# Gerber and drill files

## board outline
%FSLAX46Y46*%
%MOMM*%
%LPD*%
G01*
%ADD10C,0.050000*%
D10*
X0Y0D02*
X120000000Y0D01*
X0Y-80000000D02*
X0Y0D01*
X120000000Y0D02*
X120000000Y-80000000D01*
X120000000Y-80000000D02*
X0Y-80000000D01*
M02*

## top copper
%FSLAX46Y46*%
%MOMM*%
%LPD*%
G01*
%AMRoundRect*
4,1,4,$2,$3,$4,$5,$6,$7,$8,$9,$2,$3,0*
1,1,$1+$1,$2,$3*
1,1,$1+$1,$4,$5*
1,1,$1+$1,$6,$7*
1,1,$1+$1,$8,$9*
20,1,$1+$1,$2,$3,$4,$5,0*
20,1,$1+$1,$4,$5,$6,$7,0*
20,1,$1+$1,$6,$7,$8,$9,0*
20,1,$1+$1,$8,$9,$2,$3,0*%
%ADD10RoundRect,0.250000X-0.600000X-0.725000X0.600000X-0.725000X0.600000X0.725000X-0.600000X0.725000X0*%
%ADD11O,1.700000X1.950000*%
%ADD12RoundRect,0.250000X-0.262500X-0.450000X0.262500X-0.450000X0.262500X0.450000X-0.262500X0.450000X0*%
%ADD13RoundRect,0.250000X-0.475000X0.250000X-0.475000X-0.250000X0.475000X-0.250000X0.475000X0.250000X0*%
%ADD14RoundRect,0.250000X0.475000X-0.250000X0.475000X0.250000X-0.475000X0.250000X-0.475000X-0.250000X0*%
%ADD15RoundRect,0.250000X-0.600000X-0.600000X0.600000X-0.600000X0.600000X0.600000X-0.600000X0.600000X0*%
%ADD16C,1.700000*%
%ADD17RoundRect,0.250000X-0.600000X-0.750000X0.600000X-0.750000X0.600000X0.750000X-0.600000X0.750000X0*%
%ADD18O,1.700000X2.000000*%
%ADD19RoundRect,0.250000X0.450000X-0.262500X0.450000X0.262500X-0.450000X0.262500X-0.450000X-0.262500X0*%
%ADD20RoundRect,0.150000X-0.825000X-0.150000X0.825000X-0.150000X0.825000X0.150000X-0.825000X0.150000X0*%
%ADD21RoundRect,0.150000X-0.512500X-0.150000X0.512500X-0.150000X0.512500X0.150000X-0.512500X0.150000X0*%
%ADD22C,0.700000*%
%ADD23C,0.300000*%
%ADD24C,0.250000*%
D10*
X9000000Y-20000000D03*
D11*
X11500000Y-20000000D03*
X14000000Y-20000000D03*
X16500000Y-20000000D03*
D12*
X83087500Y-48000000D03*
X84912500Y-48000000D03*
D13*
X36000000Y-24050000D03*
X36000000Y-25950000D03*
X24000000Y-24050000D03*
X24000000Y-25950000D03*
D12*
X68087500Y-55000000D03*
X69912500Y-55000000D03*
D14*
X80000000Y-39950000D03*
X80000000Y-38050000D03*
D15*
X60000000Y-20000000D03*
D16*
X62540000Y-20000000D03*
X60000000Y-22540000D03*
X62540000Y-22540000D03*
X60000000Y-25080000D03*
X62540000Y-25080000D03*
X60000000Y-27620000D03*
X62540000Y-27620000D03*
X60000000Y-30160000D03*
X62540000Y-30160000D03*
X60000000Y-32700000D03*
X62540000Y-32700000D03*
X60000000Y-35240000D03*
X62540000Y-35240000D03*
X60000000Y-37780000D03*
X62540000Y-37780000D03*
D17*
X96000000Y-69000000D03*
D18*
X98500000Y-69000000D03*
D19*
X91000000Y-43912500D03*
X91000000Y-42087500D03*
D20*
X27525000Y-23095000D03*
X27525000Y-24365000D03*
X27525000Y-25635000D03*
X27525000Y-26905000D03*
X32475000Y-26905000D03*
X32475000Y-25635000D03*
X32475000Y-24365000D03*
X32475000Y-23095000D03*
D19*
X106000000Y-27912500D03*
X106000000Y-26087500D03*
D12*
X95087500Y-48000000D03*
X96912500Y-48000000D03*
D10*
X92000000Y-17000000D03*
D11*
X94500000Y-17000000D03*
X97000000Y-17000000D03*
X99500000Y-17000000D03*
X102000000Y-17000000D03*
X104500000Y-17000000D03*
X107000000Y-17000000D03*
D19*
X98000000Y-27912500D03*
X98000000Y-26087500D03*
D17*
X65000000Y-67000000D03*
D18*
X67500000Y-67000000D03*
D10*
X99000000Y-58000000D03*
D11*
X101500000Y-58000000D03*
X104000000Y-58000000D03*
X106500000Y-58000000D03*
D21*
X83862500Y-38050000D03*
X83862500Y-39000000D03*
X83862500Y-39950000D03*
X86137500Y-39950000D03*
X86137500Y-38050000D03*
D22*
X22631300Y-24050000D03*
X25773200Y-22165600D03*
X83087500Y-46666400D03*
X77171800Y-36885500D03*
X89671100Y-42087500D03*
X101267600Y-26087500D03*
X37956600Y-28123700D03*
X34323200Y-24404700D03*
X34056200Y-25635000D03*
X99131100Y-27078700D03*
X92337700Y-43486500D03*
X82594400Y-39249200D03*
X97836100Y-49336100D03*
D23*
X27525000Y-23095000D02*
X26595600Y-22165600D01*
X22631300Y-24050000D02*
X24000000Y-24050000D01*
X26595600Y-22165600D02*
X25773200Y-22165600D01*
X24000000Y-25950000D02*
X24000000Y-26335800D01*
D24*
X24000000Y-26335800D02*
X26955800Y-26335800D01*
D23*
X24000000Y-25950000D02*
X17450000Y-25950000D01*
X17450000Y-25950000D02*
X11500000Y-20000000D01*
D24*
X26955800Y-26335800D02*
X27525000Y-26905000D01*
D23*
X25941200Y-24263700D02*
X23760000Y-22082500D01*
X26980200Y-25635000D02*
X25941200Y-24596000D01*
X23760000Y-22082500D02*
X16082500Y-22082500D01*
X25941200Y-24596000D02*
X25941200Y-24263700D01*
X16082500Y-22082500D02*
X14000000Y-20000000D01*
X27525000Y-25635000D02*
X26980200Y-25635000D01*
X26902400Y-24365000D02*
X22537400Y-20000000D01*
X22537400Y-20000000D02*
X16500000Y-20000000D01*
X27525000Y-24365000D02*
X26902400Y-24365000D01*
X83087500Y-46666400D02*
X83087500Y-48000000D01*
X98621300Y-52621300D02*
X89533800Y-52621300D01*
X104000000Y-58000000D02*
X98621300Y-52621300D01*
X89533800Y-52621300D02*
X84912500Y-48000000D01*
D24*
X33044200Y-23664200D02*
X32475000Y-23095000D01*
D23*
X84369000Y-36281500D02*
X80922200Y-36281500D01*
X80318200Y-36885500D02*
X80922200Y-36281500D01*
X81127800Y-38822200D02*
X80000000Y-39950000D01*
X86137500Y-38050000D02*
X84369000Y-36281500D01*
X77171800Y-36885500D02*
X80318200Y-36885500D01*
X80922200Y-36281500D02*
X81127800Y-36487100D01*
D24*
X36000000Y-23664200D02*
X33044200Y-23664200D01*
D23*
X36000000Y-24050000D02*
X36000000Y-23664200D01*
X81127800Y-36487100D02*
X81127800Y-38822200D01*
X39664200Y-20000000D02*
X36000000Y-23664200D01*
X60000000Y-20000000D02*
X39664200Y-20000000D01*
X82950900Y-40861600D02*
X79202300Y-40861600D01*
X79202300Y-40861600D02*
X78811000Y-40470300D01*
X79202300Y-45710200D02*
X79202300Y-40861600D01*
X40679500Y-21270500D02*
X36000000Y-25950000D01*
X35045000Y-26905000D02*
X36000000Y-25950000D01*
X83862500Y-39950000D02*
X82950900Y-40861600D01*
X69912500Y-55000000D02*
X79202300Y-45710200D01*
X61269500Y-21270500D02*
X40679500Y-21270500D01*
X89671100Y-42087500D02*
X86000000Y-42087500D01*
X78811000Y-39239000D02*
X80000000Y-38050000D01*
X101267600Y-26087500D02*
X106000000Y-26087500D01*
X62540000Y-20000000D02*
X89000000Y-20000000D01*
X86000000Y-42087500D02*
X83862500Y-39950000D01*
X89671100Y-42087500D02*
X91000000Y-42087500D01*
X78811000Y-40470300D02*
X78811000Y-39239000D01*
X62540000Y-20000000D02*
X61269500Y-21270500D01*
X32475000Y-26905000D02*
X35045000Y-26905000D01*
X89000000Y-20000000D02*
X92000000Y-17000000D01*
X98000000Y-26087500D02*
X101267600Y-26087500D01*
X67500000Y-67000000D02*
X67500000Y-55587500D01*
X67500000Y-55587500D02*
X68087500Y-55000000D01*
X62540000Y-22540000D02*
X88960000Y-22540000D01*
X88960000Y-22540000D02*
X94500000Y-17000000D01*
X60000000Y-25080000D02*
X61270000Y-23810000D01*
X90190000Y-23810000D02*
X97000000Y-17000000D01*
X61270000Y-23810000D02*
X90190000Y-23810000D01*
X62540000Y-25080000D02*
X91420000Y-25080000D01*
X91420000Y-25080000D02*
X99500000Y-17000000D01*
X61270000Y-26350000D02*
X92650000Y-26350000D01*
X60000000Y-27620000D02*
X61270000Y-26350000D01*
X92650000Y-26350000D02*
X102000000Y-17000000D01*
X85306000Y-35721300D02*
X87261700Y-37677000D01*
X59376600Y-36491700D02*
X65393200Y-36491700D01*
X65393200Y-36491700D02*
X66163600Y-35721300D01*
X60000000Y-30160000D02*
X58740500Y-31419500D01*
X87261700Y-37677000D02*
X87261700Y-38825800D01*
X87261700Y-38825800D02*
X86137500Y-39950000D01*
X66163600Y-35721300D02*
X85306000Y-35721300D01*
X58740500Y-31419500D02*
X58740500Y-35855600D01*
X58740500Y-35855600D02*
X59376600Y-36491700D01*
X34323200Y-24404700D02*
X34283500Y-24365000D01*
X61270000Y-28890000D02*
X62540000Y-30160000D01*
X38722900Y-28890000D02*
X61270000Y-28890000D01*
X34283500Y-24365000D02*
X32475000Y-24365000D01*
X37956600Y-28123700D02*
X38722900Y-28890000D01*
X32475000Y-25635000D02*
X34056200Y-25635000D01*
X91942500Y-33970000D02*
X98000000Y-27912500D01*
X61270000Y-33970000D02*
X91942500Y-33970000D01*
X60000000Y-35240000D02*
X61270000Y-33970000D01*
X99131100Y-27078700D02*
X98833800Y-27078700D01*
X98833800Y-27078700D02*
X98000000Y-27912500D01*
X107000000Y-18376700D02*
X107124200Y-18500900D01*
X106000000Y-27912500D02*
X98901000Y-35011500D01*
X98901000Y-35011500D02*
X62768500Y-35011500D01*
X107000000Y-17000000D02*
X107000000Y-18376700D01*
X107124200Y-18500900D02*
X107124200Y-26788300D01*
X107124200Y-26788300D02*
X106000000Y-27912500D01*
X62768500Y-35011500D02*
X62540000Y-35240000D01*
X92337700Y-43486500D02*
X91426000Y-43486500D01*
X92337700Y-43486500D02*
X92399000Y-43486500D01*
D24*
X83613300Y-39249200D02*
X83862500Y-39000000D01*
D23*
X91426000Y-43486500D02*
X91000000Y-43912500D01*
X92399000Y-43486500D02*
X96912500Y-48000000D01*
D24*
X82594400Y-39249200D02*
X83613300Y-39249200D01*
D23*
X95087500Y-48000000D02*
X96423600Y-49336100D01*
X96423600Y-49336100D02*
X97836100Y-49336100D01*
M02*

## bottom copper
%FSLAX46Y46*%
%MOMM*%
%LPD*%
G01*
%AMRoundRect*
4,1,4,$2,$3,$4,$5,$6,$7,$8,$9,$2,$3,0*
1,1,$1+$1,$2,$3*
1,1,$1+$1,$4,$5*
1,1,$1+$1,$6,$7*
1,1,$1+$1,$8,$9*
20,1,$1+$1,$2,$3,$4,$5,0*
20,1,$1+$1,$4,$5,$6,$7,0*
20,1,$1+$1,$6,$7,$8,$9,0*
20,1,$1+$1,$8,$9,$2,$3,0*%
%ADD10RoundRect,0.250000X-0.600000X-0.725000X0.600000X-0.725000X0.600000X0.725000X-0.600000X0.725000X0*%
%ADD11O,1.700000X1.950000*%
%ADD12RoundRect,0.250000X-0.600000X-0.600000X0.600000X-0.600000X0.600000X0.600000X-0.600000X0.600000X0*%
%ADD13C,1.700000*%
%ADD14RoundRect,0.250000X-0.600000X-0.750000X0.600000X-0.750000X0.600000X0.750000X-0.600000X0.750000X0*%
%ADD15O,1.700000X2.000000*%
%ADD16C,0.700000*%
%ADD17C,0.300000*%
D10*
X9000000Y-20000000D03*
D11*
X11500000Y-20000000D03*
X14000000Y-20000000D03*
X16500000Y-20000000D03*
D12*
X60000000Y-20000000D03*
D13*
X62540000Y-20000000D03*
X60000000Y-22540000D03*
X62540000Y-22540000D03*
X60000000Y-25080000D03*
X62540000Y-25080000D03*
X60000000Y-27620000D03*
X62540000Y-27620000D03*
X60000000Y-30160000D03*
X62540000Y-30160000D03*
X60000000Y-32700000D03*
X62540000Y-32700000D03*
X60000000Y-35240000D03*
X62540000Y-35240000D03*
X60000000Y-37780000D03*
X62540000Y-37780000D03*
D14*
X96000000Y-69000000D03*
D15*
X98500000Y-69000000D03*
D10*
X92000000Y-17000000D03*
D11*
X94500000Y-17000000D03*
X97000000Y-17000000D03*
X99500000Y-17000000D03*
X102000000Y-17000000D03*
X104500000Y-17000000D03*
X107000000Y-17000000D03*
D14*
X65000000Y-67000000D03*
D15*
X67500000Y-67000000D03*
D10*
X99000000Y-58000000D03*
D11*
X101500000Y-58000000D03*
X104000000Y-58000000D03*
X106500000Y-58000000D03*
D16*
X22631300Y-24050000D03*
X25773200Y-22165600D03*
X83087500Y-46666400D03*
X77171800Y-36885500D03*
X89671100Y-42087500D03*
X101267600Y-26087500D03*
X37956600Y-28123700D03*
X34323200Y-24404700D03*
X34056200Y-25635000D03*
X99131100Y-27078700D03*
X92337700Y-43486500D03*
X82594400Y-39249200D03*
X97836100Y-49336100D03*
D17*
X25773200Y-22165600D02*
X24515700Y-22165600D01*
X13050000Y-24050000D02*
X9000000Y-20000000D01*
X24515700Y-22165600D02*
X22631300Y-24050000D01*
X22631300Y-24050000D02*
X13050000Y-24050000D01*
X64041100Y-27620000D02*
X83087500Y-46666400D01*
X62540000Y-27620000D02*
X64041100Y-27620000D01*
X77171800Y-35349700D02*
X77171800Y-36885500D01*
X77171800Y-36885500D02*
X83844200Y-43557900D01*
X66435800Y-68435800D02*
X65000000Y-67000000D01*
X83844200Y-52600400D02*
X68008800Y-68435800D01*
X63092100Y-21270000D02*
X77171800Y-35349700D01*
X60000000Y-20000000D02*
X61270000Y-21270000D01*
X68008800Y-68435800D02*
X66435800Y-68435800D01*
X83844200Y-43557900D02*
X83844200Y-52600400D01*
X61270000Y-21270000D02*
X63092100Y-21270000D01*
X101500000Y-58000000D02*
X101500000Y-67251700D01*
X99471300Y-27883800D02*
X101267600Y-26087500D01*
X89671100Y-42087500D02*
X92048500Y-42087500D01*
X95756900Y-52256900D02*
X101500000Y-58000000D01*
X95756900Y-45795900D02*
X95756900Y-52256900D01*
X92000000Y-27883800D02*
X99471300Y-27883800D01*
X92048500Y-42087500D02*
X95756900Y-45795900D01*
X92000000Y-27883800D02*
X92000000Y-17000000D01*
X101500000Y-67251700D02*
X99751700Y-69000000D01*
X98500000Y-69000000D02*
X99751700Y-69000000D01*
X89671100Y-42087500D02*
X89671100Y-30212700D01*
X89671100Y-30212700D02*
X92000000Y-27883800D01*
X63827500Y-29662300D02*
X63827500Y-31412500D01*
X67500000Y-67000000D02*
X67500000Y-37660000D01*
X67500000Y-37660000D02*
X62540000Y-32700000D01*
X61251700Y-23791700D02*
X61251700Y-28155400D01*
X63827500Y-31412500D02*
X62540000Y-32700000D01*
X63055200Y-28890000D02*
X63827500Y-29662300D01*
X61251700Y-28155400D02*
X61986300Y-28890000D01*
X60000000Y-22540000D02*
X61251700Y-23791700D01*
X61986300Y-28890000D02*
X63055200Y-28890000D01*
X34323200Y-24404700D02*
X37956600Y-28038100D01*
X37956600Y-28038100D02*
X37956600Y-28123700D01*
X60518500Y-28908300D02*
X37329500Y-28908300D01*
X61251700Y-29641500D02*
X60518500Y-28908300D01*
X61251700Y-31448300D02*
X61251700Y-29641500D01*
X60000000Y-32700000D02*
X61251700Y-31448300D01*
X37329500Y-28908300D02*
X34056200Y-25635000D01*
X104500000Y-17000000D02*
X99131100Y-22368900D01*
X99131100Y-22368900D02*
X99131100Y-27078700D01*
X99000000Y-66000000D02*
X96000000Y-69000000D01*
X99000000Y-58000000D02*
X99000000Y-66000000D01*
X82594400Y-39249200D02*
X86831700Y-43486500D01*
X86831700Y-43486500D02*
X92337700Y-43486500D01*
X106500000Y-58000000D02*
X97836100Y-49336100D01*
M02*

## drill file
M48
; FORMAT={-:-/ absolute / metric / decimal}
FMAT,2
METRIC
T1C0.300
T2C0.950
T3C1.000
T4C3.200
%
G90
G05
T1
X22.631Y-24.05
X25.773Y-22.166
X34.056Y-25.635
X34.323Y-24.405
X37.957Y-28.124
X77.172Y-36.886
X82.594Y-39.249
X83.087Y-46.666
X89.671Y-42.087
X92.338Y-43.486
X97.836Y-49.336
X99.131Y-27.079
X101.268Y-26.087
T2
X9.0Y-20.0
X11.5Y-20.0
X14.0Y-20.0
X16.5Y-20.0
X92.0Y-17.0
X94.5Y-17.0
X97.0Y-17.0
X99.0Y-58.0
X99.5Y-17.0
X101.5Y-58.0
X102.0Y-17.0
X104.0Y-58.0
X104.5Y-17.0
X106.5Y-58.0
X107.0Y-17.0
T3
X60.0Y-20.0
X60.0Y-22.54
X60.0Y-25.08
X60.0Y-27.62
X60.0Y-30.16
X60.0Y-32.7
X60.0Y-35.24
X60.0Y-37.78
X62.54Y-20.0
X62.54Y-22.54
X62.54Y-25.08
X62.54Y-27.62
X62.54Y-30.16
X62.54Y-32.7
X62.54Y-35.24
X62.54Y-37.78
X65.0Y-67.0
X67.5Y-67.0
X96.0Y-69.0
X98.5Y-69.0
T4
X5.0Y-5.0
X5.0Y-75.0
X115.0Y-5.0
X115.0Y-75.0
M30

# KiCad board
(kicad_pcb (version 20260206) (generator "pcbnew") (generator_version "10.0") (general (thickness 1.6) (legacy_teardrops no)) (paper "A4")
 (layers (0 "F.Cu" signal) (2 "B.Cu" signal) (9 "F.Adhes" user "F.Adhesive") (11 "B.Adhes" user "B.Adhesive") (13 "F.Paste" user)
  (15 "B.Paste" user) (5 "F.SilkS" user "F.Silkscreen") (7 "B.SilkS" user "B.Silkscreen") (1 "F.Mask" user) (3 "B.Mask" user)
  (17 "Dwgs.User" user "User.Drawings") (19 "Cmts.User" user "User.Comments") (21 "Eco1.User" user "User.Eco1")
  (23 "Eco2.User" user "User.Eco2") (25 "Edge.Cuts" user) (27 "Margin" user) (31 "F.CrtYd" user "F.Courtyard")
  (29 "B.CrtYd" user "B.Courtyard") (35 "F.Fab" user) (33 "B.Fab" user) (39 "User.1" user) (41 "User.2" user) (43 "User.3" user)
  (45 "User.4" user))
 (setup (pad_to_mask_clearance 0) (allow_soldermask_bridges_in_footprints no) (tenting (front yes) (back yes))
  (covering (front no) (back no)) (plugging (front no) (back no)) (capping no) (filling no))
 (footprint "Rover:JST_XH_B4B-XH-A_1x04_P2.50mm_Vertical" (layer "F.Cu") (at 9 20)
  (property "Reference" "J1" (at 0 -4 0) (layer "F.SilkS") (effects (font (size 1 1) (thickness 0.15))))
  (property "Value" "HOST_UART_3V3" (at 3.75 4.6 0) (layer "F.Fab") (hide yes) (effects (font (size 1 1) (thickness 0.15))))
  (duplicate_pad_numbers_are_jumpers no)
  (pad "1" thru_hole roundrect (at 0 0) (size 1.7 1.95) (drill 0.95) (layers "*.Cu" "*.Mask") (remove_unused_layers no)
   (roundrect_rratio 0.147059) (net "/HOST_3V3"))
  (pad "2" thru_hole oval (at 2.5 0) (size 1.7 1.95) (drill 0.95) (layers "*.Cu" "*.Mask") (remove_unused_layers no) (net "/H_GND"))
  (pad "3" thru_hole oval (at 5 0) (size 1.7 1.95) (drill 0.95) (layers "*.Cu" "*.Mask") (remove_unused_layers no) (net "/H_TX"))
  (pad "4" thru_hole oval (at 7.5 0) (size 1.7 1.95) (drill 0.95) (layers "*.Cu" "*.Mask") (remove_unused_layers no) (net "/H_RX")))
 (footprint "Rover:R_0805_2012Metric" (layer "F.Cu") (at 84 48)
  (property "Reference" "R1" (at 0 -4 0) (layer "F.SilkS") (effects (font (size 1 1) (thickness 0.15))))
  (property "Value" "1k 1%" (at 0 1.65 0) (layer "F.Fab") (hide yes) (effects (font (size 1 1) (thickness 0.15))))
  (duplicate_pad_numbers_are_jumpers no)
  (pad "1" smd roundrect (at -0.9125 0) (size 1.025 1.4) (layers "F.Cu" "F.Mask" "F.Paste") (roundrect_rratio 0.243902) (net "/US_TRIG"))
  (pad "2" smd roundrect (at 0.9125 0) (size 1.025 1.4) (layers "F.Cu" "F.Mask" "F.Paste") (roundrect_rratio 0.243902) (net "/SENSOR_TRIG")))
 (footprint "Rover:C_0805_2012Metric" (layer "F.Cu") (at 36 25 -90)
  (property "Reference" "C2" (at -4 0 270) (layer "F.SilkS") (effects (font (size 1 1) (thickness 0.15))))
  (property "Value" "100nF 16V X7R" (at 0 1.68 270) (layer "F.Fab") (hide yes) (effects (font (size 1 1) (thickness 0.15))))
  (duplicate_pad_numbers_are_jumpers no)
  (pad "1" smd roundrect (at -0.95 0 270) (size 1 1.45) (layers "F.Cu" "F.Mask" "F.Paste") (roundrect_rratio 0.25) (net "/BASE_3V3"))
  (pad "2" smd roundrect (at 0.95 0 270) (size 1 1.45) (layers "F.Cu" "F.Mask" "F.Paste") (roundrect_rratio 0.25) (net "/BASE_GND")))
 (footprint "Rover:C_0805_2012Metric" (layer "F.Cu") (at 24 25 -90)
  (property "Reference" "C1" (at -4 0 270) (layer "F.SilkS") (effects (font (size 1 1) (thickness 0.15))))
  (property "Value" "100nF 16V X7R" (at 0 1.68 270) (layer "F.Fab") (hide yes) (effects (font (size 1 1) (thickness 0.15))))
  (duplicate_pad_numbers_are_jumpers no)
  (pad "1" smd roundrect (at -0.95 0 270) (size 1 1.45) (layers "F.Cu" "F.Mask" "F.Paste") (roundrect_rratio 0.25) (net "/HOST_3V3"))
  (pad "2" smd roundrect (at 0.95 0 270) (size 1 1.45) (layers "F.Cu" "F.Mask" "F.Paste") (roundrect_rratio 0.25) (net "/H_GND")))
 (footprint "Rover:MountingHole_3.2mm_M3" (layer "F.Cu") (at 115 75)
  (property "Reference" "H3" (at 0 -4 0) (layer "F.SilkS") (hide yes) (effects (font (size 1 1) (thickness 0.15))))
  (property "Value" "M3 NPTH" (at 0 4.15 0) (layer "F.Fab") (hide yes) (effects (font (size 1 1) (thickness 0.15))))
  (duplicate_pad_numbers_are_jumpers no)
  (pad "" np_thru_hole circle (at 0 0) (size 3.2 3.2) (drill 3.2) (layers "*.Cu" "*.Mask")))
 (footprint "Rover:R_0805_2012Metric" (layer "F.Cu") (at 69 55)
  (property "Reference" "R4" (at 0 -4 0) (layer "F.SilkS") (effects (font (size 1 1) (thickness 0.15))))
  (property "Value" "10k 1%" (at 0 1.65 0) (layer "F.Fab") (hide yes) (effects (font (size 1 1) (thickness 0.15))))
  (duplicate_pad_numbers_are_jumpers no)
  (pad "1" smd roundrect (at -0.9125 0) (size 1.025 1.4) (layers "F.Cu" "F.Mask" "F.Paste") (roundrect_rratio 0.243902) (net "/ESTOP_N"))
  (pad "2" smd roundrect (at 0.9125 0) (size 1.025 1.4) (layers "F.Cu" "F.Mask" "F.Paste") (roundrect_rratio 0.243902) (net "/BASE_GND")))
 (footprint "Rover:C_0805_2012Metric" (layer "F.Cu") (at 80 39 90)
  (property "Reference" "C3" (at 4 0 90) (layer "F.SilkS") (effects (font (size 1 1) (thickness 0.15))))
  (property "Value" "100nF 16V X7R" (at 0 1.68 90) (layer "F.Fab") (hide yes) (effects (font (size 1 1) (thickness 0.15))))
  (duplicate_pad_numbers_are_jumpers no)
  (pad "1" smd roundrect (at -0.95 0 90) (size 1 1.45) (layers "F.Cu" "F.Mask" "F.Paste") (roundrect_rratio 0.25) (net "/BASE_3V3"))
  (pad "2" smd roundrect (at 0.95 0 90) (size 1 1.45) (layers "F.Cu" "F.Mask" "F.Paste") (roundrect_rratio 0.25) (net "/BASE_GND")))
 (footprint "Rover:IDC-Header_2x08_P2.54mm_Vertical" (layer "F.Cu") (at 60 20)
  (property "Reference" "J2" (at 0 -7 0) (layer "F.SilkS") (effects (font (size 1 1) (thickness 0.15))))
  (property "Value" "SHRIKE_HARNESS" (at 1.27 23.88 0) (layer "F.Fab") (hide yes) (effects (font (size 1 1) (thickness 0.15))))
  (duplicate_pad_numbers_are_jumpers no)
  (pad "1" thru_hole roundrect (at 0 0) (size 1.7 1.7) (drill 1) (layers "*.Cu" "*.Mask") (remove_unused_layers no)
   (roundrect_rratio 0.147059) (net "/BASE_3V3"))
  (pad "2" thru_hole circle (at 2.54 0) (size 1.7 1.7) (drill 1) (layers "*.Cu" "*.Mask") (remove_unused_layers no) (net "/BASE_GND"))
  (pad "3" thru_hole circle (at 0 2.54) (size 1.7 1.7) (drill 1) (layers "*.Cu" "*.Mask") (remove_unused_layers no) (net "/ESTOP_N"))
  (pad "4" thru_hole circle (at 2.54 2.54) (size 1.7 1.7) (drill 1) (layers "*.Cu" "*.Mask") (remove_unused_layers no) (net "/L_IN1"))
  (pad "5" thru_hole circle (at 0 5.08) (size 1.7 1.7) (drill 1) (layers "*.Cu" "*.Mask") (remove_unused_layers no) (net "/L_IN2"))
  (pad "6" thru_hole circle (at 2.54 5.08) (size 1.7 1.7) (drill 1) (layers "*.Cu" "*.Mask") (remove_unused_layers no) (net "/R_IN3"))
  (pad "7" thru_hole circle (at 0 7.62) (size 1.7 1.7) (drill 1) (layers "*.Cu" "*.Mask") (remove_unused_layers no) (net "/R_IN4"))
  (pad "8" thru_hole circle (at 2.54 7.62) (size 1.7 1.7) (drill 1) (layers "*.Cu" "*.Mask") (remove_unused_layers no) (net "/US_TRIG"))
  (pad "9" thru_hole circle (at 0 10.16) (size 1.7 1.7) (drill 1) (layers "*.Cu" "*.Mask") (remove_unused_layers no) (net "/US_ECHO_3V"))
  (pad "10" thru_hole circle (at 2.54 10.16) (size 1.7 1.7) (drill 1) (layers "*.Cu" "*.Mask") (remove_unused_layers no) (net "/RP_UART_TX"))
  (pad "11" thru_hole circle (at 0 12.7) (size 1.7 1.7) (drill 1) (layers "*.Cu" "*.Mask") (remove_unused_layers no) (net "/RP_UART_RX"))
  (pad "12" thru_hole circle (at 2.54 12.7) (size 1.7 1.7) (drill 1) (layers "*.Cu" "*.Mask") (remove_unused_layers no) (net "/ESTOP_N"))
  (pad "13" thru_hole circle (at 0 15.24) (size 1.7 1.7) (drill 1) (layers "*.Cu" "*.Mask") (remove_unused_layers no) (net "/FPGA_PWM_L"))
  (pad "14" thru_hole circle (at 2.54 15.24) (size 1.7 1.7) (drill 1) (layers "*.Cu" "*.Mask") (remove_unused_layers no) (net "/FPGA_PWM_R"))
  (pad "15" thru_hole circle (at 0 17.78) (size 1.7 1.7) (drill 1) (layers "*.Cu" "*.Mask") (remove_unused_layers no)
   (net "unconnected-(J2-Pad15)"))
  (pad "16" thru_hole circle (at 2.54 17.78) (size 1.7 1.7) (drill 1) (layers "*.Cu" "*.Mask") (remove_unused_layers no)
   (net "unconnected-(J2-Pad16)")))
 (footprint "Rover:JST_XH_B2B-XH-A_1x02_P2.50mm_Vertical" (layer "F.Cu") (at 96 69)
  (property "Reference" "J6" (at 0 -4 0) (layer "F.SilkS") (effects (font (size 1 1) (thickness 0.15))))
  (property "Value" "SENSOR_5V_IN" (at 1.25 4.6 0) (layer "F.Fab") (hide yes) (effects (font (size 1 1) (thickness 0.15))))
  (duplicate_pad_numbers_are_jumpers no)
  (pad "1" thru_hole roundrect (at 0 0) (size 1.7 2) (drill 1) (layers "*.Cu" "*.Mask") (remove_unused_layers no)
   (roundrect_rratio 0.147059) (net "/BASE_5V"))
  (pad "2" thru_hole oval (at 2.5 0) (size 1.7 2) (drill 1) (layers "*.Cu" "*.Mask") (remove_unused_layers no) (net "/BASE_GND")))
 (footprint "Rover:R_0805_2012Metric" (layer "F.Cu") (at 91 43 90)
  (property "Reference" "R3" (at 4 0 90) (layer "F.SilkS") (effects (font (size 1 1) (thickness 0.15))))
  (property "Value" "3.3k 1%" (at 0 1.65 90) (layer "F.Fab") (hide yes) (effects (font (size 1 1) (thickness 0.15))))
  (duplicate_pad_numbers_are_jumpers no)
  (pad "1" smd roundrect (at -0.9125 0 90) (size 1.025 1.4) (layers "F.Cu" "F.Mask" "F.Paste") (roundrect_rratio 0.243902) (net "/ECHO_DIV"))
  (pad "2" smd roundrect (at 0.9125 0 90) (size 1.025 1.4) (layers "F.Cu" "F.Mask" "F.Paste") (roundrect_rratio 0.243902) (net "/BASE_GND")))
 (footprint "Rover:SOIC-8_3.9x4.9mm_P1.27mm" (layer "F.Cu") (at 30 25)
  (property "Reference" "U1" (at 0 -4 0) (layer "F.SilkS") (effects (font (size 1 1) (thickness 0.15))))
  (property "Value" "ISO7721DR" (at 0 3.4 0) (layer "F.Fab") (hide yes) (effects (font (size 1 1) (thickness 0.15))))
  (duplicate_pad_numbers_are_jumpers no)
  (pad "1" smd roundrect (at -2.475 -1.905) (size 1.95 0.6) (layers "F.Cu" "F.Mask" "F.Paste") (roundrect_rratio 0.25) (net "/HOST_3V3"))
  (pad "2" smd roundrect (at -2.475 -0.635) (size 1.95 0.6) (layers "F.Cu" "F.Mask" "F.Paste") (roundrect_rratio 0.25) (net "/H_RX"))
  (pad "3" smd roundrect (at -2.475 0.635) (size 1.95 0.6) (layers "F.Cu" "F.Mask" "F.Paste") (roundrect_rratio 0.25) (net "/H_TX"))
  (pad "4" smd roundrect (at -2.475 1.905) (size 1.95 0.6) (layers "F.Cu" "F.Mask" "F.Paste") (roundrect_rratio 0.25) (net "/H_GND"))
  (pad "5" smd roundrect (at 2.475 1.905) (size 1.95 0.6) (layers "F.Cu" "F.Mask" "F.Paste") (roundrect_rratio 0.25) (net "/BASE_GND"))
  (pad "6" smd roundrect (at 2.475 0.635) (size 1.95 0.6) (layers "F.Cu" "F.Mask" "F.Paste") (roundrect_rratio 0.25) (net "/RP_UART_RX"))
  (pad "7" smd roundrect (at 2.475 -0.635) (size 1.95 0.6) (layers "F.Cu" "F.Mask" "F.Paste") (roundrect_rratio 0.25) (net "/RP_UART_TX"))
  (pad "8" smd roundrect (at 2.475 -1.905) (size 1.95 0.6) (layers "F.Cu" "F.Mask" "F.Paste") (roundrect_rratio 0.25) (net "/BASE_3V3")))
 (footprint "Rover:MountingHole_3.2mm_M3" (layer "F.Cu") (at 5 75)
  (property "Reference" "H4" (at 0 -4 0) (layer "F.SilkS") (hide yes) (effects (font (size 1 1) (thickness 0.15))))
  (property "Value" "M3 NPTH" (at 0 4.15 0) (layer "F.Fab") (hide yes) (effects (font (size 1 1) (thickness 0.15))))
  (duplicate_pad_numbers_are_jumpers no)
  (pad "" np_thru_hole circle (at 0 0) (size 3.2 3.2) (drill 3.2) (layers "*.Cu" "*.Mask")))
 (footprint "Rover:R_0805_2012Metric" (layer "F.Cu") (at 106 27 90)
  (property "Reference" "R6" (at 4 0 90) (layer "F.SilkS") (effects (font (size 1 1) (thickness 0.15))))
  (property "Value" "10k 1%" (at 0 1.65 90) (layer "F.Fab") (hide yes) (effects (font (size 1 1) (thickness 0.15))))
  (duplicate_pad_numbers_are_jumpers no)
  (pad "1" smd roundrect (at -0.9125 0 90) (size 1.025 1.4) (layers "F.Cu" "F.Mask" "F.Paste") (roundrect_rratio 0.243902)
   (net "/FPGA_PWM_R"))
  (pad "2" smd roundrect (at 0.9125 0 90) (size 1.025 1.4) (layers "F.Cu" "F.Mask" "F.Paste") (roundrect_rratio 0.243902) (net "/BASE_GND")))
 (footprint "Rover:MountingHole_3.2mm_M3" (layer "F.Cu") (at 5 5)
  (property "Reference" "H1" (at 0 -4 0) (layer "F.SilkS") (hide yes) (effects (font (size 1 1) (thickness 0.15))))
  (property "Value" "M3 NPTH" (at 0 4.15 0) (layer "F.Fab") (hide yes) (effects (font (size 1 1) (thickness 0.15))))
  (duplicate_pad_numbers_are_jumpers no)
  (pad "" np_thru_hole circle (at 0 0) (size 3.2 3.2) (drill 3.2) (layers "*.Cu" "*.Mask")))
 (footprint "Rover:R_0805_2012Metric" (layer "F.Cu") (at 96 48)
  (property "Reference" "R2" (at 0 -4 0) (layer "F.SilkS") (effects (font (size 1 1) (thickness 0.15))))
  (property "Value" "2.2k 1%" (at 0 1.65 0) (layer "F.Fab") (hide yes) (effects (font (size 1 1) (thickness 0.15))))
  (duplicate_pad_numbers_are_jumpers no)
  (pad "1" smd roundrect (at -0.9125 0) (size 1.025 1.4) (layers "F.Cu" "F.Mask" "F.Paste") (roundrect_rratio 0.243902) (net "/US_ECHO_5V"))
  (pad "2" smd roundrect (at 0.9125 0) (size 1.025 1.4) (layers "F.Cu" "F.Mask" "F.Paste") (roundrect_rratio 0.243902) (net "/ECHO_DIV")))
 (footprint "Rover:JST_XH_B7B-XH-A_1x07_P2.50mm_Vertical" (layer "F.Cu") (at 92 17)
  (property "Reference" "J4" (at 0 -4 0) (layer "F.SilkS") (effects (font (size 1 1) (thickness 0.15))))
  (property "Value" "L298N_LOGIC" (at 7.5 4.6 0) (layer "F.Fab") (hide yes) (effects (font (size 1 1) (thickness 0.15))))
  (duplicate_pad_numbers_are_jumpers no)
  (pad "1" thru_hole roundrect (at 0 0) (size 1.7 1.95) (drill 0.95) (layers "*.Cu" "*.Mask") (remove_unused_layers no)
   (roundrect_rratio 0.147059) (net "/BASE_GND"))
  (pad "2" thru_hole oval (at 2.5 0) (size 1.7 1.95) (drill 0.95) (layers "*.Cu" "*.Mask") (remove_unused_layers no) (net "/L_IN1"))
  (pad "3" thru_hole oval (at 5 0) (size 1.7 1.95) (drill 0.95) (layers "*.Cu" "*.Mask") (remove_unused_layers no) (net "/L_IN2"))
  (pad "4" thru_hole oval (at 7.5 0) (size 1.7 1.95) (drill 0.95) (layers "*.Cu" "*.Mask") (remove_unused_layers no) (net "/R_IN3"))
  (pad "5" thru_hole oval (at 10 0) (size 1.7 1.95) (drill 0.95) (layers "*.Cu" "*.Mask") (remove_unused_layers no) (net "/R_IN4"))
  (pad "6" thru_hole oval (at 12.5 0) (size 1.7 1.95) (drill 0.95) (layers "*.Cu" "*.Mask") (remove_unused_layers no) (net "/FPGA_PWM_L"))
  (pad "7" thru_hole oval (at 15 0) (size 1.7 1.95) (drill 0.95) (layers "*.Cu" "*.Mask") (remove_unused_layers no) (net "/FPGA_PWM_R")))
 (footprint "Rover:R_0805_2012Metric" (layer "F.Cu") (at 98 27 90)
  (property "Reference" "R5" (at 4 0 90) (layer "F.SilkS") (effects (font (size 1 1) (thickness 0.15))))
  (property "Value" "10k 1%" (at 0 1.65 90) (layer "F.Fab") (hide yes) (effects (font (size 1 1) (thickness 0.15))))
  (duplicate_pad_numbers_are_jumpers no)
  (pad "1" smd roundrect (at -0.9125 0 90) (size 1.025 1.4) (layers "F.Cu" "F.Mask" "F.Paste") (roundrect_rratio 0.243902)
   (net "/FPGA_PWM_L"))
  (pad "2" smd roundrect (at 0.9125 0 90) (size 1.025 1.4) (layers "F.Cu" "F.Mask" "F.Paste") (roundrect_rratio 0.243902) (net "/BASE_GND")))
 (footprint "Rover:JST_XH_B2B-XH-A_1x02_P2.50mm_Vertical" (layer "F.Cu") (at 65 67)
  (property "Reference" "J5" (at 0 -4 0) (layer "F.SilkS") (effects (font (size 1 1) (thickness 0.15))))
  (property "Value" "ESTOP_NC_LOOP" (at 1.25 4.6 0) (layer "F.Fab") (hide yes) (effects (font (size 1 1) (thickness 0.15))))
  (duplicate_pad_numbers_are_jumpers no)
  (pad "1" thru_hole roundrect (at 0 0) (size 1.7 2) (drill 1) (layers "*.Cu" "*.Mask") (remove_unused_layers no)
   (roundrect_rratio 0.147059) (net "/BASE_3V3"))
  (pad "2" thru_hole oval (at 2.5 0) (size 1.7 2) (drill 1) (layers "*.Cu" "*.Mask") (remove_unused_layers no) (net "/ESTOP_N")))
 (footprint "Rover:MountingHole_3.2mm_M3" (layer "F.Cu") (at 115 5)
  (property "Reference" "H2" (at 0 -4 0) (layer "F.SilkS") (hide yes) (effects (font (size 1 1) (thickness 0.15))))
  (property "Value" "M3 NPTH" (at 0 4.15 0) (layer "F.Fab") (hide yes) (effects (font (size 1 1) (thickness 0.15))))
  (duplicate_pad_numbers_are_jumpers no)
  (pad "" np_thru_hole circle (at 0 0) (size 3.2 3.2) (drill 3.2) (layers "*.Cu" "*.Mask")))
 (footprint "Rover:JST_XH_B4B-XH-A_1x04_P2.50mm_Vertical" (layer "F.Cu") (at 99 58)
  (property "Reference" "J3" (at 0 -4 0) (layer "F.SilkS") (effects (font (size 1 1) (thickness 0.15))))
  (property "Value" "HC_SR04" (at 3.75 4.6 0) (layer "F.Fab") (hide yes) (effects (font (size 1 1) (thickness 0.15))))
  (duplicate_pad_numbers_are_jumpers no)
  (pad "1" thru_hole roundrect (at 0 0) (size 1.7 1.95) (drill 0.95) (layers "*.Cu" "*.Mask") (remove_unused_layers no)
   (roundrect_rratio 0.147059) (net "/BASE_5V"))
  (pad "2" thru_hole oval (at 2.5 0) (size 1.7 1.95) (drill 0.95) (layers "*.Cu" "*.Mask") (remove_unused_layers no) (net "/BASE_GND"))
  (pad "3" thru_hole oval (at 5 0) (size 1.7 1.95) (drill 0.95) (layers "*.Cu" "*.Mask") (remove_unused_layers no) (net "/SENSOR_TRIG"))
  (pad "4" thru_hole oval (at 7.5 0) (size 1.7 1.95) (drill 0.95) (layers "*.Cu" "*.Mask") (remove_unused_layers no) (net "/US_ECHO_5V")))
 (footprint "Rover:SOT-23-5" (layer "F.Cu") (at 85 39)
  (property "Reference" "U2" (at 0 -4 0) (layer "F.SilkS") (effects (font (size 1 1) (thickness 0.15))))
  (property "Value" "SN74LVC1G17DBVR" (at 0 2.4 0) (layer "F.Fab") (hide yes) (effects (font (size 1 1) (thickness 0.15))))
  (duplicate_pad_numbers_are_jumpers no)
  (pad "1" smd roundrect (at -1.1375 -0.95) (size 1.325 0.6) (layers "F.Cu" "F.Mask" "F.Paste") (roundrect_rratio 0.25)
   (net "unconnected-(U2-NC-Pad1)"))
  (pad "2" smd roundrect (at -1.1375 0) (size 1.325 0.6) (layers "F.Cu" "F.Mask" "F.Paste") (roundrect_rratio 0.25) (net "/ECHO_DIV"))
  (pad "3" smd roundrect (at -1.1375 0.95) (size 1.325 0.6) (layers "F.Cu" "F.Mask" "F.Paste") (roundrect_rratio 0.25) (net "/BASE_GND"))
  (pad "4" smd roundrect (at 1.1375 0.95) (size 1.325 0.6) (layers "F.Cu" "F.Mask" "F.Paste") (roundrect_rratio 0.25) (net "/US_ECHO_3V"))
  (pad "5" smd roundrect (at 1.1375 -0.95) (size 1.325 0.6) (layers "F.Cu" "F.Mask" "F.Paste") (roundrect_rratio 0.25) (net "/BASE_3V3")))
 (gr_line (start 0 0) (end 120 0) (stroke (width 0.05) (type default)) (layer "Edge.Cuts"))
 (gr_line (start 0 80) (end 0 0) (stroke (width 0.05) (type default)) (layer "Edge.Cuts"))
 (gr_line (start 120 0) (end 120 80) (stroke (width 0.05) (type default)) (layer "Edge.Cuts"))
 (gr_line (start 120 80) (end 0 80) (stroke (width 0.05) (type default)) (layer "Edge.Cuts"))
 (segment (start 27.525 23.095) (end 26.5956 22.1656) (width 0.3) (layer "F.Cu") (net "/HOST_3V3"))
 (segment (start 22.6313 24.05) (end 24 24.05) (width 0.3) (layer "F.Cu") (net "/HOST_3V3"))
 (segment (start 26.5956 22.1656) (end 25.7732 22.1656) (width 0.3) (layer "F.Cu") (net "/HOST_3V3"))
 (via (at 22.6313 24.05) (size 0.7) (drill 0.3) (layers "F.Cu" "B.Cu") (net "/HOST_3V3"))
 (via (at 25.7732 22.1656) (size 0.7) (drill 0.3) (layers "F.Cu" "B.Cu") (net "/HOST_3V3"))
 (segment (start 25.7732 22.1656) (end 24.5157 22.1656) (width 0.3) (layer "B.Cu") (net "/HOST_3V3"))
 (segment (start 13.05 24.05) (end 9 20) (width 0.3) (layer "B.Cu") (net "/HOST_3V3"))
 (segment (start 24.5157 22.1656) (end 22.6313 24.05) (width 0.3) (layer "B.Cu") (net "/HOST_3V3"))
 (segment (start 22.6313 24.05) (end 13.05 24.05) (width 0.3) (layer "B.Cu") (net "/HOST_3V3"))
 (segment (start 24 25.95) (end 24 26.3358) (width 0.3) (layer "F.Cu") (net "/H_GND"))
 (segment (start 24 26.3358) (end 26.9558 26.3358) (width 0.25) (layer "F.Cu") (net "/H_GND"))
 (segment (start 24 25.95) (end 17.45 25.95) (width 0.3) (layer "F.Cu") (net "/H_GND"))
 (segment (start 17.45 25.95) (end 11.5 20) (width 0.3) (layer "F.Cu") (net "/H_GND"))
 (segment (start 26.9558 26.3358) (end 27.525 26.905) (width 0.25) (layer "F.Cu") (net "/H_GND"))
 (segment (start 25.9412 24.2637) (end 23.76 22.0825) (width 0.3) (layer "F.Cu") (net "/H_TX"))
 (segment (start 26.9802 25.635) (end 25.9412 24.596) (width 0.3) (layer "F.Cu") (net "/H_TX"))
 (segment (start 23.76 22.0825) (end 16.0825 22.0825) (width 0.3) (layer "F.Cu") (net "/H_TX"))
 (segment (start 25.9412 24.596) (end 25.9412 24.2637) (width 0.3) (layer "F.Cu") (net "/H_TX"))
 (segment (start 16.0825 22.0825) (end 14 20) (width 0.3) (layer "F.Cu") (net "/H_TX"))
 (segment (start 27.525 25.635) (end 26.9802 25.635) (width 0.3) (layer "F.Cu") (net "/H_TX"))
 (segment (start 26.9024 24.365) (end 22.5374 20) (width 0.3) (layer "F.Cu") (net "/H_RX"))
 (segment (start 22.5374 20) (end 16.5 20) (width 0.3) (layer "F.Cu") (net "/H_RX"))
 (segment (start 27.525 24.365) (end 26.9024 24.365) (width 0.3) (layer "F.Cu") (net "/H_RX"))
 (segment (start 83.0875 46.6664) (end 83.0875 48) (width 0.3) (layer "F.Cu") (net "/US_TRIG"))
 (via (at 83.0875 46.6664) (size 0.7) (drill 0.3) (layers "F.Cu" "B.Cu") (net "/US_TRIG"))
 (segment (start 64.0411 27.62) (end 83.0875 46.6664) (width 0.3) (layer "B.Cu") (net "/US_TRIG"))
 (segment (start 62.54 27.62) (end 64.0411 27.62) (width 0.3) (layer "B.Cu") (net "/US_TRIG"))
 (segment (start 98.6213 52.6213) (end 89.5338 52.6213) (width 0.3) (layer "F.Cu") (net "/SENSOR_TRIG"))
 (segment (start 104 58) (end 98.6213 52.6213) (width 0.3) (layer "F.Cu") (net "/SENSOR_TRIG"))
 (segment (start 89.5338 52.6213) (end 84.9125 48) (width 0.3) (layer "F.Cu") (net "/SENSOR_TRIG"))
 (segment (start 33.0442 23.6642) (end 32.475 23.095) (width 0.25) (layer "F.Cu") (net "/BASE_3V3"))
 (segment (start 84.369 36.2815) (end 80.9222 36.2815) (width 0.3) (layer "F.Cu") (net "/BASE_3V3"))
 (segment (start 80.3182 36.8855) (end 80.9222 36.2815) (width 0.3) (layer "F.Cu") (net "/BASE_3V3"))
 (segment (start 81.1278 38.8222) (end 80 39.95) (width 0.3) (layer "F.Cu") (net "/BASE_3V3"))
 (segment (start 86.1375 38.05) (end 84.369 36.2815) (width 0.3) (layer "F.Cu") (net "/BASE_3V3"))
 (segment (start 77.1718 36.8855) (end 80.3182 36.8855) (width 0.3) (layer "F.Cu") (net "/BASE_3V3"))
 (segment (start 80.9222 36.2815) (end 81.1278 36.4871) (width 0.3) (layer "F.Cu") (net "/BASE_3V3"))
 (segment (start 36 23.6642) (end 33.0442 23.6642) (width 0.25) (layer "F.Cu") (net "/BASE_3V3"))
 (segment (start 36 24.05) (end 36 23.6642) (width 0.3) (layer "F.Cu") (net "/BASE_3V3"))
 (segment (start 81.1278 36.4871) (end 81.1278 38.8222) (width 0.3) (layer "F.Cu") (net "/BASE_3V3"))
 (segment (start 39.6642 20) (end 36 23.6642) (width 0.3) (layer "F.Cu") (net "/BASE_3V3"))
 (segment (start 60 20) (end 39.6642 20) (width 0.3) (layer "F.Cu") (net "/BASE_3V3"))
 (via (at 77.1718 36.8855) (size 0.7) (drill 0.3) (layers "F.Cu" "B.Cu") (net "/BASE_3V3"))
 (segment (start 77.1718 35.3497) (end 77.1718 36.8855) (width 0.3) (layer "B.Cu") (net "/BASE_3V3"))
 (segment (start 77.1718 36.8855) (end 83.8442 43.5579) (width 0.3) (layer "B.Cu") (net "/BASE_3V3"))
 (segment (start 66.4358 68.4358) (end 65 67) (width 0.3) (layer "B.Cu") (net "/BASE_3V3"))
 (segment (start 83.8442 52.6004) (end 68.0088 68.4358) (width 0.3) (layer "B.Cu") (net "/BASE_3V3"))
 (segment (start 63.0921 21.27) (end 77.1718 35.3497) (width 0.3) (layer "B.Cu") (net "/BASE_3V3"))
 (segment (start 60 20) (end 61.27 21.27) (width 0.3) (layer "B.Cu") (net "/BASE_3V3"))
 (segment (start 68.0088 68.4358) (end 66.4358 68.4358) (width 0.3) (layer "B.Cu") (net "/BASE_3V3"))
 (segment (start 83.8442 43.5579) (end 83.8442 52.6004) (width 0.3) (layer "B.Cu") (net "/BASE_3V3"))
 (segment (start 61.27 21.27) (end 63.0921 21.27) (width 0.3) (layer "B.Cu") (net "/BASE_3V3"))
 (segment (start 82.9509 40.8616) (end 79.2023 40.8616) (width 0.3) (layer "F.Cu") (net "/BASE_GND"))
 (segment (start 79.2023 40.8616) (end 78.811 40.4703) (width 0.3) (layer "F.Cu") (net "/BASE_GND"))
 (segment (start 79.2023 45.7102) (end 79.2023 40.8616) (width 0.3) (layer "F.Cu") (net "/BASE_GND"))
 (segment (start 40.6795 21.2705) (end 36 25.95) (width 0.3) (layer "F.Cu") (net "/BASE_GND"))
 (segment (start 35.045 26.905) (end 36 25.95) (width 0.3) (layer "F.Cu") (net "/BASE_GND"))
 (segment (start 83.8625 39.95) (end 82.9509 40.8616) (width 0.3) (layer "F.Cu") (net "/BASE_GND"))
 (segment (start 69.9125 55) (end 79.2023 45.7102) (width 0.3) (layer "F.Cu") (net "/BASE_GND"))
 (segment (start 61.2695 21.2705) (end 40.6795 21.2705) (width 0.3) (layer "F.Cu") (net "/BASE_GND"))
 (segment (start 89.6711 42.0875) (end 86 42.0875) (width 0.3) (layer "F.Cu") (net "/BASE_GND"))
 (segment (start 78.811 39.239) (end 80 38.05) (width 0.3) (layer "F.Cu") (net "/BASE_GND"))
 (segment (start 101.2676 26.0875) (end 106 26.0875) (width 0.3) (layer "F.Cu") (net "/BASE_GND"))
 (segment (start 62.54 20) (end 89 20) (width 0.3) (layer "F.Cu") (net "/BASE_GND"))
 (segment (start 86 42.0875) (end 83.8625 39.95) (width 0.3) (layer "F.Cu") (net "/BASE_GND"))
 (segment (start 89.6711 42.0875) (end 91 42.0875) (width 0.3) (layer "F.Cu") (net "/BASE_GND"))
 (segment (start 78.811 40.4703) (end 78.811 39.239) (width 0.3) (layer "F.Cu") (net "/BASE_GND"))
 (segment (start 62.54 20) (end 61.2695 21.2705) (width 0.3) (layer "F.Cu") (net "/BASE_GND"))
 (segment (start 32.475 26.905) (end 35.045 26.905) (width 0.3) (layer "F.Cu") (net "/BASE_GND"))
 (segment (start 89 20) (end 92 17) (width 0.3) (layer "F.Cu") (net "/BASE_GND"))
 (segment (start 98 26.0875) (end 101.2676 26.0875) (width 0.3) (layer "F.Cu") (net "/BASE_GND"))
 (via (at 89.6711 42.0875) (size 0.7) (drill 0.3) (layers "F.Cu" "B.Cu") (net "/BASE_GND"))
 (via (at 101.2676 26.0875) (size 0.7) (drill 0.3) (layers "F.Cu" "B.Cu") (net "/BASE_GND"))
 (segment (start 101.5 58) (end 101.5 67.2517) (width 0.3) (layer "B.Cu") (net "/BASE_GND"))
 (segment (start 99.4713 27.8838) (end 101.2676 26.0875) (width 0.3) (layer "B.Cu") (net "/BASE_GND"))
 (segment (start 89.6711 42.0875) (end 92.0485 42.0875) (width 0.3) (layer "B.Cu") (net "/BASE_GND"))
 (segment (start 95.7569 52.2569) (end 101.5 58) (width 0.3) (layer "B.Cu") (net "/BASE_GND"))
 (segment (start 95.7569 45.7959) (end 95.7569 52.2569) (width 0.3) (layer "B.Cu") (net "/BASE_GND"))
 (segment (start 92 27.8838) (end 99.4713 27.8838) (width 0.3) (layer "B.Cu") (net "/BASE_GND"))
 (segment (start 92.0485 42.0875) (end 95.7569 45.7959) (width 0.3) (layer "B.Cu") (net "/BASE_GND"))
 (segment (start 92 27.8838) (end 92 17) (width 0.3) (layer "B.Cu") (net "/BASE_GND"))
 (segment (start 101.5 67.2517) (end 99.7517 69) (width 0.3) (layer "B.Cu") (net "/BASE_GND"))
 (segment (start 98.5 69) (end 99.7517 69) (width 0.3) (layer "B.Cu") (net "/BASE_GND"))
 (segment (start 89.6711 42.0875) (end 89.6711 30.2127) (width 0.3) (layer "B.Cu") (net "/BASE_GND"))
 (segment (start 89.6711 30.2127) (end 92 27.8838) (width 0.3) (layer "B.Cu") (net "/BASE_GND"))
 (segment (start 67.5 67) (end 67.5 55.5875) (width 0.3) (layer "F.Cu") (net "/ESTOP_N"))
 (segment (start 67.5 55.5875) (end 68.0875 55) (width 0.3) (layer "F.Cu") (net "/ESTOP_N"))
 (segment (start 63.8275 29.6623) (end 63.8275 31.4125) (width 0.3) (layer "B.Cu") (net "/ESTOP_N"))
 (segment (start 67.5 67) (end 67.5 37.66) (width 0.3) (layer "B.Cu") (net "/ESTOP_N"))
 (segment (start 67.5 37.66) (end 62.54 32.7) (width 0.3) (layer "B.Cu") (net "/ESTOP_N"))
 (segment (start 61.2517 23.7917) (end 61.2517 28.1554) (width 0.3) (layer "B.Cu") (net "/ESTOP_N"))
 (segment (start 63.8275 31.4125) (end 62.54 32.7) (width 0.3) (layer "B.Cu") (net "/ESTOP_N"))
 (segment (start 63.0552 28.89) (end 63.8275 29.6623) (width 0.3) (layer "B.Cu") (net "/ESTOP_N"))
 (segment (start 61.2517 28.1554) (end 61.9863 28.89) (width 0.3) (layer "B.Cu") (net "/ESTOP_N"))
 (segment (start 60 22.54) (end 61.2517 23.7917) (width 0.3) (layer "B.Cu") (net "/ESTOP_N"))
 (segment (start 61.9863 28.89) (end 63.0552 28.89) (width 0.3) (layer "B.Cu") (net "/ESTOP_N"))
 (segment (start 62.54 22.54) (end 88.96 22.54) (width 0.3) (layer "F.Cu") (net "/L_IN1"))
 (segment (start 88.96 22.54) (end 94.5 17) (width 0.3) (layer "F.Cu") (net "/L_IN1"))
 (segment (start 60 25.08) (end 61.27 23.81) (width 0.3) (layer "F.Cu") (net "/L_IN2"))
 (segment (start 90.19 23.81) (end 97 17) (width 0.3) (layer "F.Cu") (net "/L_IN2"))
 (segment (start 61.27 23.81) (end 90.19 23.81) (width 0.3) (layer "F.Cu") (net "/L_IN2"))
 (segment (start 62.54 25.08) (end 91.42 25.08) (width 0.3) (layer "F.Cu") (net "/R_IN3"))
 (segment (start 91.42 25.08) (end 99.5 17) (width 0.3) (layer "F.Cu") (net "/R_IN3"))
 (segment (start 61.27 26.35) (end 92.65 26.35) (width 0.3) (layer "F.Cu") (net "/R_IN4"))
 (segment (start 60 27.62) (end 61.27 26.35) (width 0.3) (layer "F.Cu") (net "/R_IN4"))
 (segment (start 92.65 26.35) (end 102 17) (width 0.3) (layer "F.Cu") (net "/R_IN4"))
 (segment (start 85.306 35.7213) (end 87.2617 37.677) (width 0.3) (layer "F.Cu") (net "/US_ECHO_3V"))
 (segment (start 59.3766 36.4917) (end 65.3932 36.4917) (width 0.3) (layer "F.Cu") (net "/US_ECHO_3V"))
 (segment (start 65.3932 36.4917) (end 66.1636 35.7213) (width 0.3) (layer "F.Cu") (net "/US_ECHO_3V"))
 (segment (start 60 30.16) (end 58.7405 31.4195) (width 0.3) (layer "F.Cu") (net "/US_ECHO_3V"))
 (segment (start 87.2617 37.677) (end 87.2617 38.8258) (width 0.3) (layer "F.Cu") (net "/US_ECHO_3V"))
 (segment (start 87.2617 38.8258) (end 86.1375 39.95) (width 0.3) (layer "F.Cu") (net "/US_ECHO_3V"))
 (segment (start 66.1636 35.7213) (end 85.306 35.7213) (width 0.3) (layer "F.Cu") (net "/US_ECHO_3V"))
 (segment (start 58.7405 31.4195) (end 58.7405 35.8556) (width 0.3) (layer "F.Cu") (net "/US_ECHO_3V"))
 (segment (start 58.7405 35.8556) (end 59.3766 36.4917) (width 0.3) (layer "F.Cu") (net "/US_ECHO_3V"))
 (segment (start 34.3232 24.4047) (end 34.2835 24.365) (width 0.3) (layer "F.Cu") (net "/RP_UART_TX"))
 (segment (start 61.27 28.89) (end 62.54 30.16) (width 0.3) (layer "F.Cu") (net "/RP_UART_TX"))
 (segment (start 38.7229 28.89) (end 61.27 28.89) (width 0.3) (layer "F.Cu") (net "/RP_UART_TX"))
 (segment (start 34.2835 24.365) (end 32.475 24.365) (width 0.3) (layer "F.Cu") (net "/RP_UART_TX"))
 (segment (start 37.9566 28.1237) (end 38.7229 28.89) (width 0.3) (layer "F.Cu") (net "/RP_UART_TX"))
 (via (at 37.9566 28.1237) (size 0.7) (drill 0.3) (layers "F.Cu" "B.Cu") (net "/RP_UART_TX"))
 (via (at 34.3232 24.4047) (size 0.7) (drill 0.3) (layers "F.Cu" "B.Cu") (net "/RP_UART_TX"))
 (segment (start 34.3232 24.4047) (end 37.9566 28.0381) (width 0.3) (layer "B.Cu") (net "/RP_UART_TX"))
 (segment (start 37.9566 28.0381) (end 37.9566 28.1237) (width 0.3) (layer "B.Cu") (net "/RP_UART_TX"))
 (segment (start 32.475 25.635) (end 34.0562 25.635) (width 0.3) (layer "F.Cu") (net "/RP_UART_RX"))
 (via (at 34.0562 25.635) (size 0.7) (drill 0.3) (layers "F.Cu" "B.Cu") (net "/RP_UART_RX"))
 (segment (start 60.5185 28.9083) (end 37.3295 28.9083) (width 0.3) (layer "B.Cu") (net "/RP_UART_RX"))
 (segment (start 61.2517 29.6415) (end 60.5185 28.9083) (width 0.3) (layer "B.Cu") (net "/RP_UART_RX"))
 (segment (start 61.2517 31.4483) (end 61.2517 29.6415) (width 0.3) (layer "B.Cu") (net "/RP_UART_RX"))
 (segment (start 60 32.7) (end 61.2517 31.4483) (width 0.3) (layer "B.Cu") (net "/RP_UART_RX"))
 (segment (start 37.3295 28.9083) (end 34.0562 25.635) (width 0.3) (layer "B.Cu") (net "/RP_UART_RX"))
 (segment (start 91.9425 33.97) (end 98 27.9125) (width 0.3) (layer "F.Cu") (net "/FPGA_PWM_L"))
 (segment (start 61.27 33.97) (end 91.9425 33.97) (width 0.3) (layer "F.Cu") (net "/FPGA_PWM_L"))
 (segment (start 60 35.24) (end 61.27 33.97) (width 0.3) (layer "F.Cu") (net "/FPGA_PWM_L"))
 (segment (start 99.1311 27.0787) (end 98.8338 27.0787) (width 0.3) (layer "F.Cu") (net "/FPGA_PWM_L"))
 (segment (start 98.8338 27.0787) (end 98 27.9125) (width 0.3) (layer "F.Cu") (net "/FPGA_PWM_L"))
 (via (at 99.1311 27.0787) (size 0.7) (drill 0.3) (layers "F.Cu" "B.Cu") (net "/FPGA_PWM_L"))
 (segment (start 104.5 17) (end 99.1311 22.3689) (width 0.3) (layer "B.Cu") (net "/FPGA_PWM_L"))
 (segment (start 99.1311 22.3689) (end 99.1311 27.0787) (width 0.3) (layer "B.Cu") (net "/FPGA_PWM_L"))
 (segment (start 107 18.3767) (end 107.1242 18.5009) (width 0.3) (layer "F.Cu") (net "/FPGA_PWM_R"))
 (segment (start 106 27.9125) (end 98.901 35.0115) (width 0.3) (layer "F.Cu") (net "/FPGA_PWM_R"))
 (segment (start 98.901 35.0115) (end 62.7685 35.0115) (width 0.3) (layer "F.Cu") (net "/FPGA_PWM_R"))
 (segment (start 107 17) (end 107 18.3767) (width 0.3) (layer "F.Cu") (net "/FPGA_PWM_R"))
 (segment (start 107.1242 18.5009) (end 107.1242 26.7883) (width 0.3) (layer "F.Cu") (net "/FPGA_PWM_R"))
 (segment (start 107.1242 26.7883) (end 106 27.9125) (width 0.3) (layer "F.Cu") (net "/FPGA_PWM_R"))
 (segment (start 62.7685 35.0115) (end 62.54 35.24) (width 0.3) (layer "F.Cu") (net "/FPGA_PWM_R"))
 (segment (start 99 66) (end 96 69) (width 0.3) (layer "B.Cu") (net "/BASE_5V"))
 (segment (start 99 58) (end 99 66) (width 0.3) (layer "B.Cu") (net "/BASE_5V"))
 (segment (start 92.3377 43.4865) (end 91.426 43.4865) (width 0.3) (layer "F.Cu") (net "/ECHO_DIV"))
 (segment (start 92.3377 43.4865) (end 92.399 43.4865) (width 0.3) (layer "F.Cu") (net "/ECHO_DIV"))
 (segment (start 83.6133 39.2492) (end 83.8625 39) (width 0.25) (layer "F.Cu") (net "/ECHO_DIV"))
 (segment (start 91.426 43.4865) (end 91 43.9125) (width 0.3) (layer "F.Cu") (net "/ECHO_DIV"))
 (segment (start 92.399 43.4865) (end 96.9125 48) (width 0.3) (layer "F.Cu") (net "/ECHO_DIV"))
 (segment (start 82.5944 39.2492) (end 83.6133 39.2492) (width 0.25) (layer "F.Cu") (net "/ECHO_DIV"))
 (via (at 92.3377 43.4865) (size 0.7) (drill 0.3) (layers "F.Cu" "B.Cu") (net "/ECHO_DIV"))
 (via (at 82.5944 39.2492) (size 0.7) (drill 0.3) (layers "F.Cu" "B.Cu") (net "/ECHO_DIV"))
 (segment (start 82.5944 39.2492) (end 86.8317 43.4865) (width 0.3) (layer "B.Cu") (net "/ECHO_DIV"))
 (segment (start 86.8317 43.4865) (end 92.3377 43.4865) (width 0.3) (layer "B.Cu") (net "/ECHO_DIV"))
 (segment (start 95.0875 48) (end 96.4236 49.3361) (width 0.3) (layer "F.Cu") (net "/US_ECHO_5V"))
 (segment (start 96.4236 49.3361) (end 97.8361 49.3361) (width 0.3) (layer "F.Cu") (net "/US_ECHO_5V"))
 (via (at 97.8361 49.3361) (size 0.7) (drill 0.3) (layers "F.Cu" "B.Cu") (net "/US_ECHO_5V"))
 (segment (start 106.5 58) (end 97.8361 49.3361) (width 0.3) (layer "B.Cu") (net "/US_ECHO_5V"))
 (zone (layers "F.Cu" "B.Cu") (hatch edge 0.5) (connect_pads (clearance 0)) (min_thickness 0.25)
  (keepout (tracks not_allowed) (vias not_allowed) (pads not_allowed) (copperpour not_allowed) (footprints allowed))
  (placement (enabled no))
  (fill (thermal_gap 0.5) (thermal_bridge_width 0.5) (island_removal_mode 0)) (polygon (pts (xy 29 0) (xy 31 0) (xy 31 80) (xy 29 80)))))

